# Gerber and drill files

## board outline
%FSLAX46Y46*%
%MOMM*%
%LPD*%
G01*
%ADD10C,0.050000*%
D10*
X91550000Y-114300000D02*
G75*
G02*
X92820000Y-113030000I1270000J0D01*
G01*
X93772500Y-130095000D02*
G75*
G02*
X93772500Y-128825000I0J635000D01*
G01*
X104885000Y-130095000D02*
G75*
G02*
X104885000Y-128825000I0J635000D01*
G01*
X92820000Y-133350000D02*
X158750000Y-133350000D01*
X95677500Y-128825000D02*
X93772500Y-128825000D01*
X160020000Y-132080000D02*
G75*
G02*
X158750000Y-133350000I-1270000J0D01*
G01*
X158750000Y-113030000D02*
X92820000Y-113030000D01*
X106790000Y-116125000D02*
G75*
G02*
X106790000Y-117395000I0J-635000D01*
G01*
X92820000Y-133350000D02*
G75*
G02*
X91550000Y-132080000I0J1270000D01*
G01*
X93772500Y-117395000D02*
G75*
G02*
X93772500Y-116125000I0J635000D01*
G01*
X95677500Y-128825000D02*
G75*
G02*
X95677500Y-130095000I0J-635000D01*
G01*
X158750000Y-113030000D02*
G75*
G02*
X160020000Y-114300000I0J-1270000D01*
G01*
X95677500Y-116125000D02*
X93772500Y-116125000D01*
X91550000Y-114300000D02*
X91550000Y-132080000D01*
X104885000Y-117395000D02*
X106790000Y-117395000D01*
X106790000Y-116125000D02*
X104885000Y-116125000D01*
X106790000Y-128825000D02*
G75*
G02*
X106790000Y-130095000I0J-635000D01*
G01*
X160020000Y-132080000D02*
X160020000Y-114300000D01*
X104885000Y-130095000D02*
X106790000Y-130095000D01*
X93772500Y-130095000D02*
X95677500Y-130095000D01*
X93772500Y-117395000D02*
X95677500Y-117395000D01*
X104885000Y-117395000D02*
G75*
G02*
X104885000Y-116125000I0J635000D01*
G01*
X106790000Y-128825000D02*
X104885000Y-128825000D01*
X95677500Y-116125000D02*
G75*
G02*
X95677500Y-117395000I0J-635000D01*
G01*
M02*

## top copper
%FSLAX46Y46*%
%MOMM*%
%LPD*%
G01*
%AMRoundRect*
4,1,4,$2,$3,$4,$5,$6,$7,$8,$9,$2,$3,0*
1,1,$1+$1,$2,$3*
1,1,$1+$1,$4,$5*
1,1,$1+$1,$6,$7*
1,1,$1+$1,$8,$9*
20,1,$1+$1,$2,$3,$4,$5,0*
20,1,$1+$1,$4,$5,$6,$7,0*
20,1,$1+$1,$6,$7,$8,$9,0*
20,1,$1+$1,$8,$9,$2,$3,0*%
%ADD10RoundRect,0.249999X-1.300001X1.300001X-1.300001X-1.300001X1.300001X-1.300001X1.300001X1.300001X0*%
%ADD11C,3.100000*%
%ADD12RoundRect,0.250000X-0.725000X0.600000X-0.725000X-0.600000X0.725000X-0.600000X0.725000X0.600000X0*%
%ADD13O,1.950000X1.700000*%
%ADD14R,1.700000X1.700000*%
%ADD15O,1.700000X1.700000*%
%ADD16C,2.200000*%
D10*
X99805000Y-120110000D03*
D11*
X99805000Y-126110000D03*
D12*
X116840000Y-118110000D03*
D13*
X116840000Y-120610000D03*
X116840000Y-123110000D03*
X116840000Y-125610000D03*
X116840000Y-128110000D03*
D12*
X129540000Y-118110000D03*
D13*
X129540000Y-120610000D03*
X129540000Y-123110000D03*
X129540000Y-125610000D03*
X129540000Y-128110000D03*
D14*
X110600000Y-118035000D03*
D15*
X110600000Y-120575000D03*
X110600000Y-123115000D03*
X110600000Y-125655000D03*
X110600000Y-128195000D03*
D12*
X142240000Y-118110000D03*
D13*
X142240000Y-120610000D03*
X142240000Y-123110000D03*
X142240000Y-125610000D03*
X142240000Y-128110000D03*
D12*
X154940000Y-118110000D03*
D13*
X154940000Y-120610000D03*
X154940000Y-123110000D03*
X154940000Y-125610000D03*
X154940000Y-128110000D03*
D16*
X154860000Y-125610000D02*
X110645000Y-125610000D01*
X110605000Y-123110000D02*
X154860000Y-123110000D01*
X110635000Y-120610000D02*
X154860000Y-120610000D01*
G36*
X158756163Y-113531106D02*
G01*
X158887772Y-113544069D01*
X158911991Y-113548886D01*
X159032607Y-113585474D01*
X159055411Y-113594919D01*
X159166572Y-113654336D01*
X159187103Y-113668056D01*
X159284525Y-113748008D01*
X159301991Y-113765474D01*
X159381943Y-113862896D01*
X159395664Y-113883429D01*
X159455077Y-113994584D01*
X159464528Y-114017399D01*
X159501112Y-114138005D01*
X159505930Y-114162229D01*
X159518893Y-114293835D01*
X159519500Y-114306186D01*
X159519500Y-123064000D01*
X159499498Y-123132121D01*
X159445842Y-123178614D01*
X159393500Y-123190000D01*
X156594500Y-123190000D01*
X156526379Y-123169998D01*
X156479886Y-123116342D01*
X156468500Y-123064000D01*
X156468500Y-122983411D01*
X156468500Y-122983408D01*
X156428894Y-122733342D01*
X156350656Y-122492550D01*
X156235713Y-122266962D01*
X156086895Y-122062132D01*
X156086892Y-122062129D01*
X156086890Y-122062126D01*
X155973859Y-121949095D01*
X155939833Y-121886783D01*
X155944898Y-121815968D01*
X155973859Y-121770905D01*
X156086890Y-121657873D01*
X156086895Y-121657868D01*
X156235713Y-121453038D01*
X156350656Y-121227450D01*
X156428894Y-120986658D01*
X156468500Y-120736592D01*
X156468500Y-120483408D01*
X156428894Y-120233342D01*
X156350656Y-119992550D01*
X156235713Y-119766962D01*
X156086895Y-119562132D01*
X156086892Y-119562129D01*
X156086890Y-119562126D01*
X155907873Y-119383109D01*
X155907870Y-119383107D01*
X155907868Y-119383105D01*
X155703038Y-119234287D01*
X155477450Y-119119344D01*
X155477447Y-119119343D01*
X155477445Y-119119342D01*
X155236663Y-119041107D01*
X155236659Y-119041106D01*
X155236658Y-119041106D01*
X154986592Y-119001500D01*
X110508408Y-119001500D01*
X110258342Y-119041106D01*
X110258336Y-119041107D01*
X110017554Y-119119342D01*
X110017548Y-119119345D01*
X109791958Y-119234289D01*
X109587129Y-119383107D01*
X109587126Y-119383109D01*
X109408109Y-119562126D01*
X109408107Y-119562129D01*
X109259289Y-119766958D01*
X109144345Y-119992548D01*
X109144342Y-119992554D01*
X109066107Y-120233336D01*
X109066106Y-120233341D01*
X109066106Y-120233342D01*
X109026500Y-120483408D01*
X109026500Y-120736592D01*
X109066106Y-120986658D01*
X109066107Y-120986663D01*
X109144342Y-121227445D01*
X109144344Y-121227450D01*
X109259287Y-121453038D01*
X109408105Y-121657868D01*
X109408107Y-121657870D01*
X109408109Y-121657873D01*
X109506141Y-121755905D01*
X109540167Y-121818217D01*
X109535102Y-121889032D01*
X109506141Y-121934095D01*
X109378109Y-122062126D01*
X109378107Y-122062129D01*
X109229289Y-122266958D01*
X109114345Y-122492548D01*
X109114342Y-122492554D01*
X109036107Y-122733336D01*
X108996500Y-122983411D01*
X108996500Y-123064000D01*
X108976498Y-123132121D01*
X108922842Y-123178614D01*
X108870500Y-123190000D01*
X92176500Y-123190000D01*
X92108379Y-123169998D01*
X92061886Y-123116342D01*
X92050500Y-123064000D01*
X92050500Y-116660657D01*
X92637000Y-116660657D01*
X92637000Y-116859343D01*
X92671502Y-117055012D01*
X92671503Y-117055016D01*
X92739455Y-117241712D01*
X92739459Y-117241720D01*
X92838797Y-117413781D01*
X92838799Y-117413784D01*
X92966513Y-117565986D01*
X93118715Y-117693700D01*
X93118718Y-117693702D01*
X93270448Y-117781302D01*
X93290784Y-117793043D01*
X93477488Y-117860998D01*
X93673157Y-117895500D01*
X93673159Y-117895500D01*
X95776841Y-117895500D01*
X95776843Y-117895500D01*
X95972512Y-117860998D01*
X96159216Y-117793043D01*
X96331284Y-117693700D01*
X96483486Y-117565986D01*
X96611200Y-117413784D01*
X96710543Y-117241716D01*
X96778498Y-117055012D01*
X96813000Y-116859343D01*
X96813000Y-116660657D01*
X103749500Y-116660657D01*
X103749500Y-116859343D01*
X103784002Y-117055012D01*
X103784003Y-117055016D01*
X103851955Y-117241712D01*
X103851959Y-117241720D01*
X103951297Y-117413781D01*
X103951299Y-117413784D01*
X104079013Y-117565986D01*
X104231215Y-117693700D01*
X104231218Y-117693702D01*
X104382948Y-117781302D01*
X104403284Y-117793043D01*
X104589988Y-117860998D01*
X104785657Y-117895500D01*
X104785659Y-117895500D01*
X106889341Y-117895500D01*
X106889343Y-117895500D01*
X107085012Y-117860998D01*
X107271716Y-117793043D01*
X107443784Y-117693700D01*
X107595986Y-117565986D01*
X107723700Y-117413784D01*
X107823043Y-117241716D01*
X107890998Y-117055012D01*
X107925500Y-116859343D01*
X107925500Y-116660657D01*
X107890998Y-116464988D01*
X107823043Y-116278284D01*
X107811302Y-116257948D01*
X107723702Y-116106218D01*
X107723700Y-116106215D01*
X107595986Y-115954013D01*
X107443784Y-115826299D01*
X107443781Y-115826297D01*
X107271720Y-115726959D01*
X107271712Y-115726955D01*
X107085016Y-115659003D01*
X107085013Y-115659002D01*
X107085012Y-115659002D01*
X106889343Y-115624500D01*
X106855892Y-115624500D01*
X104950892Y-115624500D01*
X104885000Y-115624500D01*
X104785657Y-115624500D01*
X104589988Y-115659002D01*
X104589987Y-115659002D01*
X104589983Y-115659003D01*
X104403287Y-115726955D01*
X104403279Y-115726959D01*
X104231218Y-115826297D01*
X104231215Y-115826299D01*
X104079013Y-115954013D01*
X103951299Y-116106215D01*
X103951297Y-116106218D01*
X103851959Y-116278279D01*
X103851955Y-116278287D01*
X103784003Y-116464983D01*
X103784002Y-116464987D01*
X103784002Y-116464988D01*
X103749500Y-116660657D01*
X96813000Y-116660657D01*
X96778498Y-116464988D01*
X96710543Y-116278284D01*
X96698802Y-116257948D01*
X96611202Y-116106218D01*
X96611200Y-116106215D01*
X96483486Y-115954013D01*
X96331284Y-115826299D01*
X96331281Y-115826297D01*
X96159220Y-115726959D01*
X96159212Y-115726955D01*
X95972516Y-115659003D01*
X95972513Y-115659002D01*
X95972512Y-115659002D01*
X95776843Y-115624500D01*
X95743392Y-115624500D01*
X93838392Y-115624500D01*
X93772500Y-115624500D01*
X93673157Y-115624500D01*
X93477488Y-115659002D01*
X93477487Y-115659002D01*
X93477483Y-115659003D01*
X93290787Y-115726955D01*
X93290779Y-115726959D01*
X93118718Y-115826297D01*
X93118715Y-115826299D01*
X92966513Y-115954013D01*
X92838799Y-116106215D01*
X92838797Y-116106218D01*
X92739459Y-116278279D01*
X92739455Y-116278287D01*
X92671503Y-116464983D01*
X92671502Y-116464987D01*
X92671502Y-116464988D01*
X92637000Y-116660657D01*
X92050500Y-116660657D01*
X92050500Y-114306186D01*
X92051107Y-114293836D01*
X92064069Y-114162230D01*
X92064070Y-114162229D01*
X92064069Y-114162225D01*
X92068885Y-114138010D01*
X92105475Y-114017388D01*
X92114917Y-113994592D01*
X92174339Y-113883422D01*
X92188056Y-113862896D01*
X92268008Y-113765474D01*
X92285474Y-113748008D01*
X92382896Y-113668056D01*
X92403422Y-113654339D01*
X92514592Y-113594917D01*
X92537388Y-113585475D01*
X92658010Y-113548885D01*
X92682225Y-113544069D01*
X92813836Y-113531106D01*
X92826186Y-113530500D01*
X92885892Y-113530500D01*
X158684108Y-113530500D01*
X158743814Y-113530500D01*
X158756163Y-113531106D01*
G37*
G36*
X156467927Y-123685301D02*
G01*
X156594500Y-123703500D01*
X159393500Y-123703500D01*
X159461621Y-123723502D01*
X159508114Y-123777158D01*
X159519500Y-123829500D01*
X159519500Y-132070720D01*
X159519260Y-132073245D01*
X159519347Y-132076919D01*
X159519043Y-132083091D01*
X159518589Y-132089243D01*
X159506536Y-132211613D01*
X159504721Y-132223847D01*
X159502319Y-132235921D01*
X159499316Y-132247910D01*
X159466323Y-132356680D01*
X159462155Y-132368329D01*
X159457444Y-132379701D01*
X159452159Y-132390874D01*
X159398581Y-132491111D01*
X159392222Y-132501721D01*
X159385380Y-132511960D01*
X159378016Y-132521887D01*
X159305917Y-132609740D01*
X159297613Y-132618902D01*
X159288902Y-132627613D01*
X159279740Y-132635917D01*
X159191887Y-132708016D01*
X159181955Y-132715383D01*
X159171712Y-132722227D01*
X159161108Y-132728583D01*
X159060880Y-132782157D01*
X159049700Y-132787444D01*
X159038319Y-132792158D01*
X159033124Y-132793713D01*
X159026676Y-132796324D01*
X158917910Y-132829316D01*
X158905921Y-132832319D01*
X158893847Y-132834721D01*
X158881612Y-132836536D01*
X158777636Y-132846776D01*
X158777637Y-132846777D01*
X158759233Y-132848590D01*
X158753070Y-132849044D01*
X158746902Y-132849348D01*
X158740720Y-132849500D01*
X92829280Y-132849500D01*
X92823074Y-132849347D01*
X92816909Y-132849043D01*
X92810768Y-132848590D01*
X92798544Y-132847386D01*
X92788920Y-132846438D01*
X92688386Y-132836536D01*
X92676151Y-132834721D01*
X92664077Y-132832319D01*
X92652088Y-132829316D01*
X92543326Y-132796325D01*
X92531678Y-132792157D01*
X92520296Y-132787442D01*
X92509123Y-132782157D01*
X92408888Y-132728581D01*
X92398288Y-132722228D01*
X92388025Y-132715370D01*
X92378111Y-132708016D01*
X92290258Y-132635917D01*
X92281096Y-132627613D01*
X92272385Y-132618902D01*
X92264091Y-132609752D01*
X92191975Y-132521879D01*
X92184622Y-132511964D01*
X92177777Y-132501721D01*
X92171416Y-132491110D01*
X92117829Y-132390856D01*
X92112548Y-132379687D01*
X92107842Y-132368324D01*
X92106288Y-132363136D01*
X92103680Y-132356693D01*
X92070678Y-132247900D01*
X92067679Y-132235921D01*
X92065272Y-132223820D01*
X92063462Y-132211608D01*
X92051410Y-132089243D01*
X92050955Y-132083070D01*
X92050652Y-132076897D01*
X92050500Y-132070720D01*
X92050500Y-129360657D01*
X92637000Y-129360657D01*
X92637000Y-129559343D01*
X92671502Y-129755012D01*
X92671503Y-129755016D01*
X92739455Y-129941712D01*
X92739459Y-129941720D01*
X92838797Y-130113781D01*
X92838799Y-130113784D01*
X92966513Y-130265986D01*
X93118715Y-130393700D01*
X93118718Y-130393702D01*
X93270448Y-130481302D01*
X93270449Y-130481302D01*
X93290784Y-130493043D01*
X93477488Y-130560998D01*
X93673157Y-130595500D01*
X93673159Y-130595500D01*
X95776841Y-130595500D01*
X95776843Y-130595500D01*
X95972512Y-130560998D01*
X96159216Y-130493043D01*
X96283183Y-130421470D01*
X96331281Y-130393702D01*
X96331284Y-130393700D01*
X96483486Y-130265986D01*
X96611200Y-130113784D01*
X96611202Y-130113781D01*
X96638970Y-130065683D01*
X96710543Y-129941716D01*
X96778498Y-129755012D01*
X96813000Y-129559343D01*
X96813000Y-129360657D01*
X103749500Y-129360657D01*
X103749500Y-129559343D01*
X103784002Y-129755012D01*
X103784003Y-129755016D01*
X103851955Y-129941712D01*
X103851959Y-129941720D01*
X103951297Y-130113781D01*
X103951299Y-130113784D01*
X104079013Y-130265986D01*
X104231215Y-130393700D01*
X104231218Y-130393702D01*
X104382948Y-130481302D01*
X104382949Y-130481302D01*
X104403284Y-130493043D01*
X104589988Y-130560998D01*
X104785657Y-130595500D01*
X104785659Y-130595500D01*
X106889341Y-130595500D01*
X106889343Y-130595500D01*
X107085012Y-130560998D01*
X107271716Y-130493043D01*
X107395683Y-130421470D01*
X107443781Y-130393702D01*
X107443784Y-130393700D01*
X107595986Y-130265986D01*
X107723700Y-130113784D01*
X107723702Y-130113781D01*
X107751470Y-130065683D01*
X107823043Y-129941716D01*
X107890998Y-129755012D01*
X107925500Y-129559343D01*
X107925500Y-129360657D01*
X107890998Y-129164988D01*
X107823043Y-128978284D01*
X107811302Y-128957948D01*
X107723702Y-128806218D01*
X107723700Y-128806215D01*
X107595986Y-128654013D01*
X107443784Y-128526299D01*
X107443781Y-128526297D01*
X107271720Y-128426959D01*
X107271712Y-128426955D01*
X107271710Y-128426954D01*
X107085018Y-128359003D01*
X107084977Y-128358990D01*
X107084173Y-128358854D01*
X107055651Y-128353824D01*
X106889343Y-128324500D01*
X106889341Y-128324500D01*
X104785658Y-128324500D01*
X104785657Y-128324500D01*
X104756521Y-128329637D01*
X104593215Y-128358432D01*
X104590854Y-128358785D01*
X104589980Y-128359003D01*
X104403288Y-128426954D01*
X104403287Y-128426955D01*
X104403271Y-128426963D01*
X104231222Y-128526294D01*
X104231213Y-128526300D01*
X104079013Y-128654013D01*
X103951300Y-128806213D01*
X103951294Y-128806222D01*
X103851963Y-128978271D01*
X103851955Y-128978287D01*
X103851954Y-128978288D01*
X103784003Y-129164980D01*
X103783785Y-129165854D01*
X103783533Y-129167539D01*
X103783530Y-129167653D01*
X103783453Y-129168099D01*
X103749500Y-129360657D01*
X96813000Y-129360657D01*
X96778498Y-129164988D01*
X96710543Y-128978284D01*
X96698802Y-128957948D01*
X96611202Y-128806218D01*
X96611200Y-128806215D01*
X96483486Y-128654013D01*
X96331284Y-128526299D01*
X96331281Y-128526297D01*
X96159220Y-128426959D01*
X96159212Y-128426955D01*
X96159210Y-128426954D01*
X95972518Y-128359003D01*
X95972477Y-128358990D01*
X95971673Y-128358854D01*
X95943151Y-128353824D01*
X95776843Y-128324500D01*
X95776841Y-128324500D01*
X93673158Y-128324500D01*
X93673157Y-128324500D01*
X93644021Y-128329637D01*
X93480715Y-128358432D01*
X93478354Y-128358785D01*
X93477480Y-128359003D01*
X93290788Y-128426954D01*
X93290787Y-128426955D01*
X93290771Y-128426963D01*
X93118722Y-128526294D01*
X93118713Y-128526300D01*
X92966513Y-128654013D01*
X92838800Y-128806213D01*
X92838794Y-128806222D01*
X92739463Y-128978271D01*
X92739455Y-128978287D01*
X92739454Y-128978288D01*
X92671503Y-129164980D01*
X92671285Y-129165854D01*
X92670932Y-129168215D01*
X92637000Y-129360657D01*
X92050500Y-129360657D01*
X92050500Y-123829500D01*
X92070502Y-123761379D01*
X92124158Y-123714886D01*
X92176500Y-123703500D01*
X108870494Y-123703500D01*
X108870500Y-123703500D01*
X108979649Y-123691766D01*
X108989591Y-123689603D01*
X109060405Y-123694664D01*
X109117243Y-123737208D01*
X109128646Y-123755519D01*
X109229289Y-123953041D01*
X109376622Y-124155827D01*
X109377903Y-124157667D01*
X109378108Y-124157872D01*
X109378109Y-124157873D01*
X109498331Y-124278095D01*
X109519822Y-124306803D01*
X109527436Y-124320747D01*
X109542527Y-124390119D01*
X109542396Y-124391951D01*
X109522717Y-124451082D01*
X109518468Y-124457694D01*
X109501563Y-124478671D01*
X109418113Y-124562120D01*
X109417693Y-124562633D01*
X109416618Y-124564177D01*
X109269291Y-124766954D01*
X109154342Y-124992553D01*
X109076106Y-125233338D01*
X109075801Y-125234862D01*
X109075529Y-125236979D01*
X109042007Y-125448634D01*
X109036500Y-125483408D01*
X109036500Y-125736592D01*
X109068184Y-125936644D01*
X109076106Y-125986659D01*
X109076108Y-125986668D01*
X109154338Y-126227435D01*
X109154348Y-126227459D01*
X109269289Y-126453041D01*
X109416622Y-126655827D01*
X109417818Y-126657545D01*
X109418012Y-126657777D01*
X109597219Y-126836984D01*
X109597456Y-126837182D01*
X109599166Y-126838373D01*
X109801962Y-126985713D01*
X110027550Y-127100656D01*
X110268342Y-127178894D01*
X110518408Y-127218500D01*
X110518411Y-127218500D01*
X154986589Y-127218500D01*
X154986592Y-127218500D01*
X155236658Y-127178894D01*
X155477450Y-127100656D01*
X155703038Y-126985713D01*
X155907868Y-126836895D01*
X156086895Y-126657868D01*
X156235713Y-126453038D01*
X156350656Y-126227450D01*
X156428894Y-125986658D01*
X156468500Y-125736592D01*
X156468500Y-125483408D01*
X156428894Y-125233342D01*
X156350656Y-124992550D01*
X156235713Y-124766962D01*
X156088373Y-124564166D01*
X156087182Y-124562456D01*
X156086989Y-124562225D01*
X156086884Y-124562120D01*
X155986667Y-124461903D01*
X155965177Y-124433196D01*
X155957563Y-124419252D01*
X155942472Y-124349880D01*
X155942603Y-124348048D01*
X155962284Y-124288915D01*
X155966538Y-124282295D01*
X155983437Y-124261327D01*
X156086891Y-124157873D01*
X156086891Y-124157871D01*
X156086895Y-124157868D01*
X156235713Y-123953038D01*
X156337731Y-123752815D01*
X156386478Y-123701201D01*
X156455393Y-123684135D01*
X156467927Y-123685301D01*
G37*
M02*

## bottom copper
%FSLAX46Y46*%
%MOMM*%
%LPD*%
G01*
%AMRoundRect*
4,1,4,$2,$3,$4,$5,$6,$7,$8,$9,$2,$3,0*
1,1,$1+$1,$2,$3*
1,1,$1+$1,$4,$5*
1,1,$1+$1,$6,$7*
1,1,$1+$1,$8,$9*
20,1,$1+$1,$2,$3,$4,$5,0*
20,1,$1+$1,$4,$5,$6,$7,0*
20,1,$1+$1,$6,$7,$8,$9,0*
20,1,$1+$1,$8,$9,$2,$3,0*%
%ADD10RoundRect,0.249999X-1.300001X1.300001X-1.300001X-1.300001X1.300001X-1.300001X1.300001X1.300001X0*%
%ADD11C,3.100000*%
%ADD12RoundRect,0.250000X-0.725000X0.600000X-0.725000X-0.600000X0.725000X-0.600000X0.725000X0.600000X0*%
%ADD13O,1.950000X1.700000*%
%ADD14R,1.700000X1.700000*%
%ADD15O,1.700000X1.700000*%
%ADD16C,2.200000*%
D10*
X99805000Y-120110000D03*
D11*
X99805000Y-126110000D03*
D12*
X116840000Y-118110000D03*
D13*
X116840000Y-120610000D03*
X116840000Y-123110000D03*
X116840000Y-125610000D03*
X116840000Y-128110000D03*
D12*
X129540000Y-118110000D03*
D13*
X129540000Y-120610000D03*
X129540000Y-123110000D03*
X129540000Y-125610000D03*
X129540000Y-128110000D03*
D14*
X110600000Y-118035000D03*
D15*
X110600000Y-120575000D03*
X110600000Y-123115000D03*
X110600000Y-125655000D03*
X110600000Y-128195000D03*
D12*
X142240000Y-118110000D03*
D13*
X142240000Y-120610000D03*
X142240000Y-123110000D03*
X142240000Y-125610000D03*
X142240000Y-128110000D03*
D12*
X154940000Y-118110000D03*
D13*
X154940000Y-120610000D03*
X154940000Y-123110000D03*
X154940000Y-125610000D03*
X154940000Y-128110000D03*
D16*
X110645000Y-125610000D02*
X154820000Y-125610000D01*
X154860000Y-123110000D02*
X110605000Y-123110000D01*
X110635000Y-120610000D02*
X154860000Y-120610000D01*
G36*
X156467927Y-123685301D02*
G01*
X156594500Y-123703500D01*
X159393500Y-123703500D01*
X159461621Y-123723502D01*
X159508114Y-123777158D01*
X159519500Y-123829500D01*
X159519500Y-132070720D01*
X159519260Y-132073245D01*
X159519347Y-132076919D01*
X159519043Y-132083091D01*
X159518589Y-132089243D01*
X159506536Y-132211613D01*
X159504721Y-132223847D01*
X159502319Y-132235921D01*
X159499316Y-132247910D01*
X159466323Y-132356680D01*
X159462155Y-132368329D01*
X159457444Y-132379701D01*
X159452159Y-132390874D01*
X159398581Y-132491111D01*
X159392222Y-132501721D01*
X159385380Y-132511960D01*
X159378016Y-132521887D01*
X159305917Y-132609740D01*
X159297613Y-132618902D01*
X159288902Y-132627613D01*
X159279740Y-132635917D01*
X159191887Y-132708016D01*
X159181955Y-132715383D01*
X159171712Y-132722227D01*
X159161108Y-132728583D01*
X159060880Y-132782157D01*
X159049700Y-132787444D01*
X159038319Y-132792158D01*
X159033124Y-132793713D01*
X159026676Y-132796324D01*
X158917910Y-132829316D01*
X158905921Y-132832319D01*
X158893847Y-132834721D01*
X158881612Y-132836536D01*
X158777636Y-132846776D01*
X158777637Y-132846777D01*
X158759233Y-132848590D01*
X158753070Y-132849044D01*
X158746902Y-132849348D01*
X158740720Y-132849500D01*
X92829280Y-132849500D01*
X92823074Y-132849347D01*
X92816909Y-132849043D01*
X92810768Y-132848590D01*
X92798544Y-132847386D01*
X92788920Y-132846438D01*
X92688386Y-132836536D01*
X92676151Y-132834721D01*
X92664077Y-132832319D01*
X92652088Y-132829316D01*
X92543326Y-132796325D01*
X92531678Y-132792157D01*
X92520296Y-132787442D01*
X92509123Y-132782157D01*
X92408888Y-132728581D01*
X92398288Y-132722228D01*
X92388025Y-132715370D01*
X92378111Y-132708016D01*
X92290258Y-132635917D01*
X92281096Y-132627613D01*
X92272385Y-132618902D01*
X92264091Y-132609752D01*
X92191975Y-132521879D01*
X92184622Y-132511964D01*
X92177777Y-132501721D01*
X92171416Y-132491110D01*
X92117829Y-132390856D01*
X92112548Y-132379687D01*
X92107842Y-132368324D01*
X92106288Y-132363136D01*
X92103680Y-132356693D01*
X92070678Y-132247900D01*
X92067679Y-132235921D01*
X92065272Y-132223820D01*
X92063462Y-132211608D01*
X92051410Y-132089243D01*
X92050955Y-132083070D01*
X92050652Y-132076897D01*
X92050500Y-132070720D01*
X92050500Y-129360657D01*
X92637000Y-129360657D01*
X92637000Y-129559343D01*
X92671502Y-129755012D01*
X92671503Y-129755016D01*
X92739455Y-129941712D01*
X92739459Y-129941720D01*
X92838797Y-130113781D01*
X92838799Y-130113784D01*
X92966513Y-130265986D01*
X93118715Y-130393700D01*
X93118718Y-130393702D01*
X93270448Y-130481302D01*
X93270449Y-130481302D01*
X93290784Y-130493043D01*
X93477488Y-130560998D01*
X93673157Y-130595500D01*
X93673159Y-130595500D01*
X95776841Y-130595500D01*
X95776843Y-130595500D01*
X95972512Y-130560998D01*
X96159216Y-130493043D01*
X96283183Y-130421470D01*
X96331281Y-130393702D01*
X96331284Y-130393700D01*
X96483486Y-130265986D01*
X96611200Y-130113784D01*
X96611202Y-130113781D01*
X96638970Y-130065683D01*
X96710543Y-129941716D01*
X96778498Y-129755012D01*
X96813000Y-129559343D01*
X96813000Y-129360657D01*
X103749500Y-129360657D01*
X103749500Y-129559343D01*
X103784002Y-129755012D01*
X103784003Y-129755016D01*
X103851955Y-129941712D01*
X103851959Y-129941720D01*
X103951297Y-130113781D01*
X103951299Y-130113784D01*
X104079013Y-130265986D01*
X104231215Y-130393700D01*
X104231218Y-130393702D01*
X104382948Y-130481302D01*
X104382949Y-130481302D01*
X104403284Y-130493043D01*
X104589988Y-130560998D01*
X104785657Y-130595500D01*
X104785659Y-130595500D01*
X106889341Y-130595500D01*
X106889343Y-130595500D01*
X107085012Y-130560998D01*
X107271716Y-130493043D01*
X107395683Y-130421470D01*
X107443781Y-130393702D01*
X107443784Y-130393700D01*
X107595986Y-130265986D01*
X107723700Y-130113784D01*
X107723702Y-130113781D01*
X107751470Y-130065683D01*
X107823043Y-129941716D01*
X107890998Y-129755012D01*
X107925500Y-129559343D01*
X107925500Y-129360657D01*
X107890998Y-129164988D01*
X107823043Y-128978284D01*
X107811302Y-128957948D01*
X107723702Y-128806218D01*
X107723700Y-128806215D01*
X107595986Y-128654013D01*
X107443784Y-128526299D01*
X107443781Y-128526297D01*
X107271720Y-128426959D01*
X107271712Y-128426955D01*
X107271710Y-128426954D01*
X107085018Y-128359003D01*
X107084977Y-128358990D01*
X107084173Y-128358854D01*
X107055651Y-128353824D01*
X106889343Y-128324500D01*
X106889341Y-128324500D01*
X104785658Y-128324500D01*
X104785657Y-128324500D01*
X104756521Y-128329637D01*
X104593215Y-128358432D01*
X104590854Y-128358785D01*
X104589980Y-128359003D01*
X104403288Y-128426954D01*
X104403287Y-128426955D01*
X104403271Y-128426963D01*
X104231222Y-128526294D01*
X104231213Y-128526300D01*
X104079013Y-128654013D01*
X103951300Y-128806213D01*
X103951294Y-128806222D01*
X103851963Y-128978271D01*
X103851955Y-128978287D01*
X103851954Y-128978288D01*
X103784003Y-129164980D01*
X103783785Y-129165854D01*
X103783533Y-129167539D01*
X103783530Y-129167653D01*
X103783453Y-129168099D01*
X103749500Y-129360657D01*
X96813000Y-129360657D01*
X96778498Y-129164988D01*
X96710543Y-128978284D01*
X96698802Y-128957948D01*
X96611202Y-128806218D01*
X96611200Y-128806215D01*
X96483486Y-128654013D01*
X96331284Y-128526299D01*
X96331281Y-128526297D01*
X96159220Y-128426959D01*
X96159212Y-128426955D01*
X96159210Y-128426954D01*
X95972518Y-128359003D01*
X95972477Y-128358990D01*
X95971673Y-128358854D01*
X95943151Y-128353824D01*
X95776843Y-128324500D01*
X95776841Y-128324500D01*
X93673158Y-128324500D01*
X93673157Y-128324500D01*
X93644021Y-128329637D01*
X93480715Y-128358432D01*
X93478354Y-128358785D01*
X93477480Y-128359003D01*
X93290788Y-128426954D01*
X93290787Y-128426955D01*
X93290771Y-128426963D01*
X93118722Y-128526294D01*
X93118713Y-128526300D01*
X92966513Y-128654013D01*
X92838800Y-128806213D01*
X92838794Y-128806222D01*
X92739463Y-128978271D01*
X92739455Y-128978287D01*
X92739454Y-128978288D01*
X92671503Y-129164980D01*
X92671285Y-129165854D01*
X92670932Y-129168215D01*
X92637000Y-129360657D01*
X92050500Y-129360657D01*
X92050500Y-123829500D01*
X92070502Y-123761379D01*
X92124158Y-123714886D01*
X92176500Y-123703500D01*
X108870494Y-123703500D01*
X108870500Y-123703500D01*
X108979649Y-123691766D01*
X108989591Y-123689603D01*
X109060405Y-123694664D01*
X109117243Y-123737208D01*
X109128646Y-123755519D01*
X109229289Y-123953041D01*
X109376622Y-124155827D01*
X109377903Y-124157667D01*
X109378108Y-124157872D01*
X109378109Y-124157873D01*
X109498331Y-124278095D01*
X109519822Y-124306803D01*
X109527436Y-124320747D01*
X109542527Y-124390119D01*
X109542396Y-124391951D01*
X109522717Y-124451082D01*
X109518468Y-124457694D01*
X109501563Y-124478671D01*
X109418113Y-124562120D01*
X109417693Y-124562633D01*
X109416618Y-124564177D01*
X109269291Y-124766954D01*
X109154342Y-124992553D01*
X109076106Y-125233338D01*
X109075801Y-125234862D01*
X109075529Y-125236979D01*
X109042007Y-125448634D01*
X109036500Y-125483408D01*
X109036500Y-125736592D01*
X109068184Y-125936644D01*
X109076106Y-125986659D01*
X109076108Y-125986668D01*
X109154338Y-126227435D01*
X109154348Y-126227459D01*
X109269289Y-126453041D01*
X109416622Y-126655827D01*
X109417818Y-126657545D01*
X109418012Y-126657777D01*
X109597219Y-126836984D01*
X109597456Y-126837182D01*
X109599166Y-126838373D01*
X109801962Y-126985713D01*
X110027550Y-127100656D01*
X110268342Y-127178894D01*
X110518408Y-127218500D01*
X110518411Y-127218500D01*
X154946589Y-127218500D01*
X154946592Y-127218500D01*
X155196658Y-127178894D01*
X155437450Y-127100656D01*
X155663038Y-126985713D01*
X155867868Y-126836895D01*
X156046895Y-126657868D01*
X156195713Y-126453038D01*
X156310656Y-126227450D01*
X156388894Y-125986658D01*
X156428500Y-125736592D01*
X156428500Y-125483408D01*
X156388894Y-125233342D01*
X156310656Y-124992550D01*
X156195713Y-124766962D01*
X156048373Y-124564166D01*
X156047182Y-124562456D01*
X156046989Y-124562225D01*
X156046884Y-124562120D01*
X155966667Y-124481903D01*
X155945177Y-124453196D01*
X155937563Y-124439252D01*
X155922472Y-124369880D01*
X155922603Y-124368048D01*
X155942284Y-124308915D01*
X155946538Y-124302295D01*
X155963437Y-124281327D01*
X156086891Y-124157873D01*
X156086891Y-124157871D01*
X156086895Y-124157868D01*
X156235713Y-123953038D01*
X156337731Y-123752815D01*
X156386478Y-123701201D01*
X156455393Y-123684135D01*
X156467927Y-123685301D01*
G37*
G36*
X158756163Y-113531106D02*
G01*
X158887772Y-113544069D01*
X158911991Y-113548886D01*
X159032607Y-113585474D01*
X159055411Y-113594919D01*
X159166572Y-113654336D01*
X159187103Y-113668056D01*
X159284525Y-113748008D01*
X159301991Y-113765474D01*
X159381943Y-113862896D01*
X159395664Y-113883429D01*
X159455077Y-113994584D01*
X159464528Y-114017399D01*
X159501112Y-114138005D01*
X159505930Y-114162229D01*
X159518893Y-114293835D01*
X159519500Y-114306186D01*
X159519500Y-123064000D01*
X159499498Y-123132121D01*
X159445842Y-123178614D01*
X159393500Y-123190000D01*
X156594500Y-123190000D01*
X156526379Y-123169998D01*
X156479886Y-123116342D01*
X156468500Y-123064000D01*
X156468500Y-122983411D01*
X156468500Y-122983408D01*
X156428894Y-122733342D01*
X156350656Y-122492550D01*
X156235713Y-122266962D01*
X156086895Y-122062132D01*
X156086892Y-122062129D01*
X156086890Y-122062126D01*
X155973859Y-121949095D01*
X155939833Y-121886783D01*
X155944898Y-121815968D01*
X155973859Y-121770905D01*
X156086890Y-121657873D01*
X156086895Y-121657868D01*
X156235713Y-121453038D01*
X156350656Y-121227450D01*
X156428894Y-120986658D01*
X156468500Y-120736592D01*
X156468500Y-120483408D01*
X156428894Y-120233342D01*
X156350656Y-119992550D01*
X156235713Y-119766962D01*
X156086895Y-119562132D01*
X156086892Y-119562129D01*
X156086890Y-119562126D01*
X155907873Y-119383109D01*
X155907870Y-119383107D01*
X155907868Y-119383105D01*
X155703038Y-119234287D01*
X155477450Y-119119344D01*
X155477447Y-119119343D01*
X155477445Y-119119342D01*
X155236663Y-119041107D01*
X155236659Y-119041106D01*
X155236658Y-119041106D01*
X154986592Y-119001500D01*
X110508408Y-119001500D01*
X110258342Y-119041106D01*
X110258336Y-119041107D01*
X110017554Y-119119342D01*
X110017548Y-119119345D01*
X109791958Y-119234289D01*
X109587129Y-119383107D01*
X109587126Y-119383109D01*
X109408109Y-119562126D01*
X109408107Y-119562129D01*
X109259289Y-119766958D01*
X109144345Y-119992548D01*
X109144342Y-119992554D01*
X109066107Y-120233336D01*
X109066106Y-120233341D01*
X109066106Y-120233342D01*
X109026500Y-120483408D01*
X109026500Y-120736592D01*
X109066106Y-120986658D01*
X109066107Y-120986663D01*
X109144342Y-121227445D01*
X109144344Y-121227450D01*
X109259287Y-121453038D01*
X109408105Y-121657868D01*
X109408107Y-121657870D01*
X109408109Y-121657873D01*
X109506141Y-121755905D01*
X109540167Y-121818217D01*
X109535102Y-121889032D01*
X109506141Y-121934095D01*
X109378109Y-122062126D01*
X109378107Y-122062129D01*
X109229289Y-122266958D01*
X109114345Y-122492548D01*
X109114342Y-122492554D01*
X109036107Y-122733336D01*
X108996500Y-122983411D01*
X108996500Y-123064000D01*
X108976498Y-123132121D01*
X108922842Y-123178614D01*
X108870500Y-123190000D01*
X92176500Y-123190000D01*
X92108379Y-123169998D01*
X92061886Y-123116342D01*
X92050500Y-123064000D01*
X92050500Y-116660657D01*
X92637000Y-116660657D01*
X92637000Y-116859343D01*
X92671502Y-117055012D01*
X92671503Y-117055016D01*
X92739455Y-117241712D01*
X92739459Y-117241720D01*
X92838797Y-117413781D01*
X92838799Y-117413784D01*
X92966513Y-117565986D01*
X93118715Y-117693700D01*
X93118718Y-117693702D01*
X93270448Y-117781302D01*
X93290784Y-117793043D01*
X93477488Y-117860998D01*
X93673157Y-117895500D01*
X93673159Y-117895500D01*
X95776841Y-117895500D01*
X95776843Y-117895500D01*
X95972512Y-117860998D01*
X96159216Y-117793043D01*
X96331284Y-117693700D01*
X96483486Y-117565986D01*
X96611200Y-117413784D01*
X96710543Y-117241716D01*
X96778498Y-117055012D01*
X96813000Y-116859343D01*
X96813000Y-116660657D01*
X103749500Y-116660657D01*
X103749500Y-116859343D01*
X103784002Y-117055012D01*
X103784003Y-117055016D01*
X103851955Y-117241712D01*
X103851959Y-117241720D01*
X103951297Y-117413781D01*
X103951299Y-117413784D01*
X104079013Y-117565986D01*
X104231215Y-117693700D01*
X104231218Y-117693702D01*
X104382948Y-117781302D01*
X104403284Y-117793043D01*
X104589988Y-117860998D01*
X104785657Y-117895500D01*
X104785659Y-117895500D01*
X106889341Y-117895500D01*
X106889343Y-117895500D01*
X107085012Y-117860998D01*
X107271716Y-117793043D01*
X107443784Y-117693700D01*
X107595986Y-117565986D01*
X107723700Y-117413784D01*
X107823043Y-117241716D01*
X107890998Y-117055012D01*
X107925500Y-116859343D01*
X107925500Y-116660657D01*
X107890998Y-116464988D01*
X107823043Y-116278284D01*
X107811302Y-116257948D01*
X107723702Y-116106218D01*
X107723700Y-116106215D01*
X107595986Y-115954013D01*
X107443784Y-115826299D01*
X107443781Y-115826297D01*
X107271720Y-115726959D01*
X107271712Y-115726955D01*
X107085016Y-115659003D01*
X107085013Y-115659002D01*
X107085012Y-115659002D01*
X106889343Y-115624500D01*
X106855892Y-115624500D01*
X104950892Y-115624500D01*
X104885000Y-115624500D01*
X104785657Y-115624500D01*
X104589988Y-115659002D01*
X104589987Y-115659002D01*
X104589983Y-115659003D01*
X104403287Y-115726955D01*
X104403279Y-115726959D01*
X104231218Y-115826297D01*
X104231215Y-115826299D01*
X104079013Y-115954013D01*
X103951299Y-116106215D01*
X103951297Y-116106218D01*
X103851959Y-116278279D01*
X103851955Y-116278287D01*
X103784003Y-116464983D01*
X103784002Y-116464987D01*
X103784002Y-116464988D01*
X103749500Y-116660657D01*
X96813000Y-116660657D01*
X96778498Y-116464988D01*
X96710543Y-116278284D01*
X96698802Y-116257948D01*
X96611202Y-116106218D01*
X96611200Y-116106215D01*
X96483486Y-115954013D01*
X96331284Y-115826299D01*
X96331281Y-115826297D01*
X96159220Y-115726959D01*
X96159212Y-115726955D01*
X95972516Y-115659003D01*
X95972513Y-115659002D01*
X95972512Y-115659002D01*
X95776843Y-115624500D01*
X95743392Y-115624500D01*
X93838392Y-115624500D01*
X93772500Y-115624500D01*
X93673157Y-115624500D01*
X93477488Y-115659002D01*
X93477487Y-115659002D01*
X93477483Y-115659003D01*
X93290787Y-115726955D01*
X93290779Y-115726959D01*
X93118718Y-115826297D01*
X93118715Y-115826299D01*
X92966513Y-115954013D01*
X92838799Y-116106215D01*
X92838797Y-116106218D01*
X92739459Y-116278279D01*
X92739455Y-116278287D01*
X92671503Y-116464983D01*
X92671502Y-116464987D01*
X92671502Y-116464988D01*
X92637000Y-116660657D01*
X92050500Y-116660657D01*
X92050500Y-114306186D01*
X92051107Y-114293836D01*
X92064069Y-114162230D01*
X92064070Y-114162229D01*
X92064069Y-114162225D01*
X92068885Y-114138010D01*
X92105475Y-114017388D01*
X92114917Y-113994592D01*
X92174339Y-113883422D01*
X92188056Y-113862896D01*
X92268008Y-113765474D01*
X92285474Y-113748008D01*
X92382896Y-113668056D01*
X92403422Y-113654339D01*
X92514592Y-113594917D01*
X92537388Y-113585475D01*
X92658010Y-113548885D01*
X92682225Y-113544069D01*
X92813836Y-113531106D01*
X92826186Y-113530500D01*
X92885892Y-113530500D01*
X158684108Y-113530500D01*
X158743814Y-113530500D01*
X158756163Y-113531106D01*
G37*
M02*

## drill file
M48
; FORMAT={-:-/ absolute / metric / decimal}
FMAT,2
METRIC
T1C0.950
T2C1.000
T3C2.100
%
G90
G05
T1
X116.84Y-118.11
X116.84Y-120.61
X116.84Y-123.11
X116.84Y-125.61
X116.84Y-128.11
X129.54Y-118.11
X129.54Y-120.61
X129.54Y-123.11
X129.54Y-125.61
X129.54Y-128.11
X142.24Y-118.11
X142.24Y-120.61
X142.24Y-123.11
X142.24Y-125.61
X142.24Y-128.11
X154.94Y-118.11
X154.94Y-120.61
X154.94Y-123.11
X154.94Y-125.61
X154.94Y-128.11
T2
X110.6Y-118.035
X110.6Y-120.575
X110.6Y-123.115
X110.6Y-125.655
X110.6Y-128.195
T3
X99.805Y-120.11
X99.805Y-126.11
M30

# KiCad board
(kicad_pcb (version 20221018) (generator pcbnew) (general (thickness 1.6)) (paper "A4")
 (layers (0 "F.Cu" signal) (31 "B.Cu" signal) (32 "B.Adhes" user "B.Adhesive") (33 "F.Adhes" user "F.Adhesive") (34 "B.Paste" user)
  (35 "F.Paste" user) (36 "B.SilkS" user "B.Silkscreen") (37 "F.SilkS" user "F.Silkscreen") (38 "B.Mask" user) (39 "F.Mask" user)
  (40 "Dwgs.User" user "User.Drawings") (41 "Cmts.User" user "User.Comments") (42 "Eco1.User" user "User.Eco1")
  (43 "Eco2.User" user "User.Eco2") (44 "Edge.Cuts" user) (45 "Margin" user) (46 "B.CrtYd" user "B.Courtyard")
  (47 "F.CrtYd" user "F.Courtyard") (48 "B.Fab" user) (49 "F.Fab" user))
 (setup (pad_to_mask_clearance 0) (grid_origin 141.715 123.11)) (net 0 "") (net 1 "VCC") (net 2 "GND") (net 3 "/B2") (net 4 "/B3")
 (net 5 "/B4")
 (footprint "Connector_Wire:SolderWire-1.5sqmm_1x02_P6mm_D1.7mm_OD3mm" (layer "F.Cu") (at 99.805 120.11 -90)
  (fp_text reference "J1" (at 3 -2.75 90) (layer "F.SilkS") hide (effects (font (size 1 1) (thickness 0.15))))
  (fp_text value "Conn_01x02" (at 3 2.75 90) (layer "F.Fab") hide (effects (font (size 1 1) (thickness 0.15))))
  (pad "1" thru_hole roundrect (at 0 0 270) (size 3.1 3.1) (drill 2.1) (layers "*.Cu" "*.Mask") (roundrect_rratio 0.08064483871)
   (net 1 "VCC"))
  (pad "2" thru_hole circle (at 6 0 270) (size 3.1 3.1) (drill 2.1) (layers "*.Cu" "*.Mask") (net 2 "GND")))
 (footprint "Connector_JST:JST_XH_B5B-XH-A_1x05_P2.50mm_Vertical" (layer "F.Cu") (at 116.84 118.11 -90)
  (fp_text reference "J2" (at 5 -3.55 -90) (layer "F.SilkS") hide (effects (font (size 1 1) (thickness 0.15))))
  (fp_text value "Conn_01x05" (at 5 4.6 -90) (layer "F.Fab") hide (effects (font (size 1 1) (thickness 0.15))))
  (pad "1" thru_hole roundrect (at 0 0 270) (size 1.7 1.95) (drill 0.95) (layers "*.Cu" "*.Mask") (roundrect_rratio 0.1470588235)
   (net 1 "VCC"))
  (pad "2" thru_hole oval (at 2.5 0 270) (size 1.7 1.95) (drill 0.95) (layers "*.Cu" "*.Mask") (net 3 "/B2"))
  (pad "3" thru_hole oval (at 5 0 270) (size 1.7 1.95) (drill 0.95) (layers "*.Cu" "*.Mask") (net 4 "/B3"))
  (pad "4" thru_hole oval (at 7.5 0 270) (size 1.7 1.95) (drill 0.95) (layers "*.Cu" "*.Mask") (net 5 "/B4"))
  (pad "5" thru_hole oval (at 10 0 270) (size 1.7 1.95) (drill 0.95) (layers "*.Cu" "*.Mask") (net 2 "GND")))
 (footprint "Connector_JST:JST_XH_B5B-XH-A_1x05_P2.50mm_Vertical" (layer "F.Cu") (at 129.54 118.11 -90)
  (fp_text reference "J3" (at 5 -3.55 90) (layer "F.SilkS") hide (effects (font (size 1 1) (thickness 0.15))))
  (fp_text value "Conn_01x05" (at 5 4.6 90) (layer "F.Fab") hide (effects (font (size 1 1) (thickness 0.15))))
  (pad "1" thru_hole roundrect (at 0 0 270) (size 1.7 1.95) (drill 0.95) (layers "*.Cu" "*.Mask") (roundrect_rratio 0.1470588235)
   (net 1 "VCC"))
  (pad "2" thru_hole oval (at 2.5 0 270) (size 1.7 1.95) (drill 0.95) (layers "*.Cu" "*.Mask") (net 3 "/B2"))
  (pad "3" thru_hole oval (at 5 0 270) (size 1.7 1.95) (drill 0.95) (layers "*.Cu" "*.Mask") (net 4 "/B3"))
  (pad "4" thru_hole oval (at 7.5 0 270) (size 1.7 1.95) (drill 0.95) (layers "*.Cu" "*.Mask") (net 5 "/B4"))
  (pad "5" thru_hole oval (at 10 0 270) (size 1.7 1.95) (drill 0.95) (layers "*.Cu" "*.Mask") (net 2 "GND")))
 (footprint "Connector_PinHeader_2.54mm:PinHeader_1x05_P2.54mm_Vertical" (layer "F.Cu") (at 110.6 118.035)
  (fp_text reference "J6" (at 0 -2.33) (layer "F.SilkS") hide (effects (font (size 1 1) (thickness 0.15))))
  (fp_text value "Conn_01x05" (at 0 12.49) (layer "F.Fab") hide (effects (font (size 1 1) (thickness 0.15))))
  (pad "1" thru_hole rect (at 0 0) (size 1.7 1.7) (drill 1) (layers "*.Cu" "*.Mask") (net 1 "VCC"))
  (pad "2" thru_hole oval (at 0 2.54) (size 1.7 1.7) (drill 1) (layers "*.Cu" "*.Mask") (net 3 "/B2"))
  (pad "3" thru_hole oval (at 0 5.08) (size 1.7 1.7) (drill 1) (layers "*.Cu" "*.Mask") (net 4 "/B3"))
  (pad "4" thru_hole oval (at 0 7.62) (size 1.7 1.7) (drill 1) (layers "*.Cu" "*.Mask") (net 5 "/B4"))
  (pad "5" thru_hole oval (at 0 10.16) (size 1.7 1.7) (drill 1) (layers "*.Cu" "*.Mask") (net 2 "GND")))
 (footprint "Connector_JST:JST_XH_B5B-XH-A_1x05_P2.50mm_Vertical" (layer "F.Cu") (at 142.24 118.11 -90)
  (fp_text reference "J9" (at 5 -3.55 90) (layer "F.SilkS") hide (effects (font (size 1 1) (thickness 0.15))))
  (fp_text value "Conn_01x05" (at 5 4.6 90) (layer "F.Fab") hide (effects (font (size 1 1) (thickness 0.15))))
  (pad "1" thru_hole roundrect (at 0 0 270) (size 1.7 1.95) (drill 0.95) (layers "*.Cu" "*.Mask") (roundrect_rratio 0.1470588235)
   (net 1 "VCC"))
  (pad "2" thru_hole oval (at 2.5 0 270) (size 1.7 1.95) (drill 0.95) (layers "*.Cu" "*.Mask") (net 3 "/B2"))
  (pad "3" thru_hole oval (at 5 0 270) (size 1.7 1.95) (drill 0.95) (layers "*.Cu" "*.Mask") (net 4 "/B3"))
  (pad "4" thru_hole oval (at 7.5 0 270) (size 1.7 1.95) (drill 0.95) (layers "*.Cu" "*.Mask") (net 5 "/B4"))
  (pad "5" thru_hole oval (at 10 0 270) (size 1.7 1.95) (drill 0.95) (layers "*.Cu" "*.Mask") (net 2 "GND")))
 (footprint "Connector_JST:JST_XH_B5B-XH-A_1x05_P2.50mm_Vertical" (layer "F.Cu") (at 154.94 118.11 -90)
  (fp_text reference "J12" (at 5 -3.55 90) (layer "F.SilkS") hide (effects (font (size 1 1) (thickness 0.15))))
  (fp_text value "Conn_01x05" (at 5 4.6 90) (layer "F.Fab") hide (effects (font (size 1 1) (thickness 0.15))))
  (pad "1" thru_hole roundrect (at 0 0 270) (size 1.7 1.95) (drill 0.95) (layers "*.Cu" "*.Mask") (roundrect_rratio 0.1470588235)
   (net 1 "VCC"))
  (pad "2" thru_hole oval (at 2.5 0 270) (size 1.7 1.95) (drill 0.95) (layers "*.Cu" "*.Mask") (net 3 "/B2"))
  (pad "3" thru_hole oval (at 5 0 270) (size 1.7 1.95) (drill 0.95) (layers "*.Cu" "*.Mask") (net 4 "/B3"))
  (pad "4" thru_hole oval (at 7.5 0 270) (size 1.7 1.95) (drill 0.95) (layers "*.Cu" "*.Mask") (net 5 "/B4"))
  (pad "5" thru_hole oval (at 10 0 270) (size 1.7 1.95) (drill 0.95) (layers "*.Cu" "*.Mask") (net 2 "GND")))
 (gr_arc (start 91.55 114.3) (mid 91.921974 113.401974) (end 92.82 113.03) (stroke (width 0.05) (type default)) (layer "Edge.Cuts"))
 (gr_arc (start 93.7725 130.095) (mid 93.1375 129.46) (end 93.7725 128.825) (stroke (width 0.05) (type default)) (layer "Edge.Cuts"))
 (gr_arc (start 104.885 130.095) (mid 104.25 129.46) (end 104.885 128.825) (stroke (width 0.05) (type default)) (layer "Edge.Cuts"))
 (gr_line (start 92.82 133.35) (end 158.75 133.35) (stroke (width 0.05) (type default)) (layer "Edge.Cuts"))
 (gr_line (start 95.6775 128.825) (end 93.7725 128.825) (stroke (width 0.05) (type default)) (layer "Edge.Cuts"))
 (gr_arc (start 160.02 132.08) (mid 159.648026 132.978026) (end 158.75 133.35) (stroke (width 0.05) (type default)) (layer "Edge.Cuts"))
 (gr_line (start 158.75 113.03) (end 92.82 113.03) (stroke (width 0.05) (type default)) (layer "Edge.Cuts"))
 (gr_arc (start 106.79 116.125) (mid 107.425 116.76) (end 106.79 117.395) (stroke (width 0.05) (type default)) (layer "Edge.Cuts"))
 (gr_arc (start 92.82 133.35) (mid 91.921974 132.978026) (end 91.55 132.08) (stroke (width 0.05) (type default)) (layer "Edge.Cuts"))
 (gr_arc (start 93.7725 117.395) (mid 93.1375 116.76) (end 93.7725 116.125) (stroke (width 0.05) (type default)) (layer "Edge.Cuts"))
 (gr_arc (start 95.6775 128.825) (mid 96.3125 129.46) (end 95.6775 130.095) (stroke (width 0.05) (type default)) (layer "Edge.Cuts"))
 (gr_arc (start 158.75 113.03) (mid 159.648026 113.401974) (end 160.02 114.3) (stroke (width 0.05) (type default)) (layer "Edge.Cuts"))
 (gr_line (start 95.6775 116.125) (end 93.7725 116.125) (stroke (width 0.05) (type default)) (layer "Edge.Cuts"))
 (gr_line (start 91.55 114.3) (end 91.55 132.08) (stroke (width 0.05) (type default)) (layer "Edge.Cuts"))
 (gr_line (start 104.885 117.395) (end 106.79 117.395) (stroke (width 0.05) (type default)) (layer "Edge.Cuts"))
 (gr_line (start 106.79 116.125) (end 104.885 116.125) (stroke (width 0.05) (type default)) (layer "Edge.Cuts"))
 (gr_arc (start 106.79 128.825) (mid 107.425 129.46) (end 106.79 130.095) (stroke (width 0.05) (type default)) (layer "Edge.Cuts"))
 (gr_line (start 160.02 132.08) (end 160.02 114.3) (stroke (width 0.05) (type default)) (layer "Edge.Cuts"))
 (gr_line (start 104.885 130.095) (end 106.79 130.095) (stroke (width 0.05) (type default)) (layer "Edge.Cuts"))
 (gr_line (start 93.7725 130.095) (end 95.6775 130.095) (stroke (width 0.05) (type default)) (layer "Edge.Cuts"))
 (gr_line (start 93.7725 117.395) (end 95.6775 117.395) (stroke (width 0.05) (type default)) (layer "Edge.Cuts"))
 (gr_arc (start 104.885 117.395) (mid 104.25 116.76) (end 104.885 116.125) (stroke (width 0.05) (type default)) (layer "Edge.Cuts"))
 (gr_line (start 106.79 128.825) (end 104.885 128.825) (stroke (width 0.05) (type default)) (layer "Edge.Cuts"))
 (gr_arc (start 95.6775 116.125) (mid 96.3125 116.76) (end 95.6775 117.395) (stroke (width 0.05) (type default)) (layer "Edge.Cuts"))
 (segment (start 154.86 125.61) (end 110.645 125.61) (width 2.2) (layer "F.Cu") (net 5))
 (segment (start 110.645 125.61) (end 154.82 125.61) (width 2.2) (layer "B.Cu") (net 5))
 (segment (start 110.605 123.11) (end 154.86 123.11) (width 2.2) (layer "F.Cu") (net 4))
 (segment (start 154.86 123.11) (end 110.605 123.11) (width 2.2) (layer "B.Cu") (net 4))
 (segment (start 110.635 120.61) (end 154.86 120.61) (width 2.2) (layer "F.Cu") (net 3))
 (segment (start 110.635 120.61) (end 154.86 120.61) (width 2.2) (layer "B.Cu") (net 3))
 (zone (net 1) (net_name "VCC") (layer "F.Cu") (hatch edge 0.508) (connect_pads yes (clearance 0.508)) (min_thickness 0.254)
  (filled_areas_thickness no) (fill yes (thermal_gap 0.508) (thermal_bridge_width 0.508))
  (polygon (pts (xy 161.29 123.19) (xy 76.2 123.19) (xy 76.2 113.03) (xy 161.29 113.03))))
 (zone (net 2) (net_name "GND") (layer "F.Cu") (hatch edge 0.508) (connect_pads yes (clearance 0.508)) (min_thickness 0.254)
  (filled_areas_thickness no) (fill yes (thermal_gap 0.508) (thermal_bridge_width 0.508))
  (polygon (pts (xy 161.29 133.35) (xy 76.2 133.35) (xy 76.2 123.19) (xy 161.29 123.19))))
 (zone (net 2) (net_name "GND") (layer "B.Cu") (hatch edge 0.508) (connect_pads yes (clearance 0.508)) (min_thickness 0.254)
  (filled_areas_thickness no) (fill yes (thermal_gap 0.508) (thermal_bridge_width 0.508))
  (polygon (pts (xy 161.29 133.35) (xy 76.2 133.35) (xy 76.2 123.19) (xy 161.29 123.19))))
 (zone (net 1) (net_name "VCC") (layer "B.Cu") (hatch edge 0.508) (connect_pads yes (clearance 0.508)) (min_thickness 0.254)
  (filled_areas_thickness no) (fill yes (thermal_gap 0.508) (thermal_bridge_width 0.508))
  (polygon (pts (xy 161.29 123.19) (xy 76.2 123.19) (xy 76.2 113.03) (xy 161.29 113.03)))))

